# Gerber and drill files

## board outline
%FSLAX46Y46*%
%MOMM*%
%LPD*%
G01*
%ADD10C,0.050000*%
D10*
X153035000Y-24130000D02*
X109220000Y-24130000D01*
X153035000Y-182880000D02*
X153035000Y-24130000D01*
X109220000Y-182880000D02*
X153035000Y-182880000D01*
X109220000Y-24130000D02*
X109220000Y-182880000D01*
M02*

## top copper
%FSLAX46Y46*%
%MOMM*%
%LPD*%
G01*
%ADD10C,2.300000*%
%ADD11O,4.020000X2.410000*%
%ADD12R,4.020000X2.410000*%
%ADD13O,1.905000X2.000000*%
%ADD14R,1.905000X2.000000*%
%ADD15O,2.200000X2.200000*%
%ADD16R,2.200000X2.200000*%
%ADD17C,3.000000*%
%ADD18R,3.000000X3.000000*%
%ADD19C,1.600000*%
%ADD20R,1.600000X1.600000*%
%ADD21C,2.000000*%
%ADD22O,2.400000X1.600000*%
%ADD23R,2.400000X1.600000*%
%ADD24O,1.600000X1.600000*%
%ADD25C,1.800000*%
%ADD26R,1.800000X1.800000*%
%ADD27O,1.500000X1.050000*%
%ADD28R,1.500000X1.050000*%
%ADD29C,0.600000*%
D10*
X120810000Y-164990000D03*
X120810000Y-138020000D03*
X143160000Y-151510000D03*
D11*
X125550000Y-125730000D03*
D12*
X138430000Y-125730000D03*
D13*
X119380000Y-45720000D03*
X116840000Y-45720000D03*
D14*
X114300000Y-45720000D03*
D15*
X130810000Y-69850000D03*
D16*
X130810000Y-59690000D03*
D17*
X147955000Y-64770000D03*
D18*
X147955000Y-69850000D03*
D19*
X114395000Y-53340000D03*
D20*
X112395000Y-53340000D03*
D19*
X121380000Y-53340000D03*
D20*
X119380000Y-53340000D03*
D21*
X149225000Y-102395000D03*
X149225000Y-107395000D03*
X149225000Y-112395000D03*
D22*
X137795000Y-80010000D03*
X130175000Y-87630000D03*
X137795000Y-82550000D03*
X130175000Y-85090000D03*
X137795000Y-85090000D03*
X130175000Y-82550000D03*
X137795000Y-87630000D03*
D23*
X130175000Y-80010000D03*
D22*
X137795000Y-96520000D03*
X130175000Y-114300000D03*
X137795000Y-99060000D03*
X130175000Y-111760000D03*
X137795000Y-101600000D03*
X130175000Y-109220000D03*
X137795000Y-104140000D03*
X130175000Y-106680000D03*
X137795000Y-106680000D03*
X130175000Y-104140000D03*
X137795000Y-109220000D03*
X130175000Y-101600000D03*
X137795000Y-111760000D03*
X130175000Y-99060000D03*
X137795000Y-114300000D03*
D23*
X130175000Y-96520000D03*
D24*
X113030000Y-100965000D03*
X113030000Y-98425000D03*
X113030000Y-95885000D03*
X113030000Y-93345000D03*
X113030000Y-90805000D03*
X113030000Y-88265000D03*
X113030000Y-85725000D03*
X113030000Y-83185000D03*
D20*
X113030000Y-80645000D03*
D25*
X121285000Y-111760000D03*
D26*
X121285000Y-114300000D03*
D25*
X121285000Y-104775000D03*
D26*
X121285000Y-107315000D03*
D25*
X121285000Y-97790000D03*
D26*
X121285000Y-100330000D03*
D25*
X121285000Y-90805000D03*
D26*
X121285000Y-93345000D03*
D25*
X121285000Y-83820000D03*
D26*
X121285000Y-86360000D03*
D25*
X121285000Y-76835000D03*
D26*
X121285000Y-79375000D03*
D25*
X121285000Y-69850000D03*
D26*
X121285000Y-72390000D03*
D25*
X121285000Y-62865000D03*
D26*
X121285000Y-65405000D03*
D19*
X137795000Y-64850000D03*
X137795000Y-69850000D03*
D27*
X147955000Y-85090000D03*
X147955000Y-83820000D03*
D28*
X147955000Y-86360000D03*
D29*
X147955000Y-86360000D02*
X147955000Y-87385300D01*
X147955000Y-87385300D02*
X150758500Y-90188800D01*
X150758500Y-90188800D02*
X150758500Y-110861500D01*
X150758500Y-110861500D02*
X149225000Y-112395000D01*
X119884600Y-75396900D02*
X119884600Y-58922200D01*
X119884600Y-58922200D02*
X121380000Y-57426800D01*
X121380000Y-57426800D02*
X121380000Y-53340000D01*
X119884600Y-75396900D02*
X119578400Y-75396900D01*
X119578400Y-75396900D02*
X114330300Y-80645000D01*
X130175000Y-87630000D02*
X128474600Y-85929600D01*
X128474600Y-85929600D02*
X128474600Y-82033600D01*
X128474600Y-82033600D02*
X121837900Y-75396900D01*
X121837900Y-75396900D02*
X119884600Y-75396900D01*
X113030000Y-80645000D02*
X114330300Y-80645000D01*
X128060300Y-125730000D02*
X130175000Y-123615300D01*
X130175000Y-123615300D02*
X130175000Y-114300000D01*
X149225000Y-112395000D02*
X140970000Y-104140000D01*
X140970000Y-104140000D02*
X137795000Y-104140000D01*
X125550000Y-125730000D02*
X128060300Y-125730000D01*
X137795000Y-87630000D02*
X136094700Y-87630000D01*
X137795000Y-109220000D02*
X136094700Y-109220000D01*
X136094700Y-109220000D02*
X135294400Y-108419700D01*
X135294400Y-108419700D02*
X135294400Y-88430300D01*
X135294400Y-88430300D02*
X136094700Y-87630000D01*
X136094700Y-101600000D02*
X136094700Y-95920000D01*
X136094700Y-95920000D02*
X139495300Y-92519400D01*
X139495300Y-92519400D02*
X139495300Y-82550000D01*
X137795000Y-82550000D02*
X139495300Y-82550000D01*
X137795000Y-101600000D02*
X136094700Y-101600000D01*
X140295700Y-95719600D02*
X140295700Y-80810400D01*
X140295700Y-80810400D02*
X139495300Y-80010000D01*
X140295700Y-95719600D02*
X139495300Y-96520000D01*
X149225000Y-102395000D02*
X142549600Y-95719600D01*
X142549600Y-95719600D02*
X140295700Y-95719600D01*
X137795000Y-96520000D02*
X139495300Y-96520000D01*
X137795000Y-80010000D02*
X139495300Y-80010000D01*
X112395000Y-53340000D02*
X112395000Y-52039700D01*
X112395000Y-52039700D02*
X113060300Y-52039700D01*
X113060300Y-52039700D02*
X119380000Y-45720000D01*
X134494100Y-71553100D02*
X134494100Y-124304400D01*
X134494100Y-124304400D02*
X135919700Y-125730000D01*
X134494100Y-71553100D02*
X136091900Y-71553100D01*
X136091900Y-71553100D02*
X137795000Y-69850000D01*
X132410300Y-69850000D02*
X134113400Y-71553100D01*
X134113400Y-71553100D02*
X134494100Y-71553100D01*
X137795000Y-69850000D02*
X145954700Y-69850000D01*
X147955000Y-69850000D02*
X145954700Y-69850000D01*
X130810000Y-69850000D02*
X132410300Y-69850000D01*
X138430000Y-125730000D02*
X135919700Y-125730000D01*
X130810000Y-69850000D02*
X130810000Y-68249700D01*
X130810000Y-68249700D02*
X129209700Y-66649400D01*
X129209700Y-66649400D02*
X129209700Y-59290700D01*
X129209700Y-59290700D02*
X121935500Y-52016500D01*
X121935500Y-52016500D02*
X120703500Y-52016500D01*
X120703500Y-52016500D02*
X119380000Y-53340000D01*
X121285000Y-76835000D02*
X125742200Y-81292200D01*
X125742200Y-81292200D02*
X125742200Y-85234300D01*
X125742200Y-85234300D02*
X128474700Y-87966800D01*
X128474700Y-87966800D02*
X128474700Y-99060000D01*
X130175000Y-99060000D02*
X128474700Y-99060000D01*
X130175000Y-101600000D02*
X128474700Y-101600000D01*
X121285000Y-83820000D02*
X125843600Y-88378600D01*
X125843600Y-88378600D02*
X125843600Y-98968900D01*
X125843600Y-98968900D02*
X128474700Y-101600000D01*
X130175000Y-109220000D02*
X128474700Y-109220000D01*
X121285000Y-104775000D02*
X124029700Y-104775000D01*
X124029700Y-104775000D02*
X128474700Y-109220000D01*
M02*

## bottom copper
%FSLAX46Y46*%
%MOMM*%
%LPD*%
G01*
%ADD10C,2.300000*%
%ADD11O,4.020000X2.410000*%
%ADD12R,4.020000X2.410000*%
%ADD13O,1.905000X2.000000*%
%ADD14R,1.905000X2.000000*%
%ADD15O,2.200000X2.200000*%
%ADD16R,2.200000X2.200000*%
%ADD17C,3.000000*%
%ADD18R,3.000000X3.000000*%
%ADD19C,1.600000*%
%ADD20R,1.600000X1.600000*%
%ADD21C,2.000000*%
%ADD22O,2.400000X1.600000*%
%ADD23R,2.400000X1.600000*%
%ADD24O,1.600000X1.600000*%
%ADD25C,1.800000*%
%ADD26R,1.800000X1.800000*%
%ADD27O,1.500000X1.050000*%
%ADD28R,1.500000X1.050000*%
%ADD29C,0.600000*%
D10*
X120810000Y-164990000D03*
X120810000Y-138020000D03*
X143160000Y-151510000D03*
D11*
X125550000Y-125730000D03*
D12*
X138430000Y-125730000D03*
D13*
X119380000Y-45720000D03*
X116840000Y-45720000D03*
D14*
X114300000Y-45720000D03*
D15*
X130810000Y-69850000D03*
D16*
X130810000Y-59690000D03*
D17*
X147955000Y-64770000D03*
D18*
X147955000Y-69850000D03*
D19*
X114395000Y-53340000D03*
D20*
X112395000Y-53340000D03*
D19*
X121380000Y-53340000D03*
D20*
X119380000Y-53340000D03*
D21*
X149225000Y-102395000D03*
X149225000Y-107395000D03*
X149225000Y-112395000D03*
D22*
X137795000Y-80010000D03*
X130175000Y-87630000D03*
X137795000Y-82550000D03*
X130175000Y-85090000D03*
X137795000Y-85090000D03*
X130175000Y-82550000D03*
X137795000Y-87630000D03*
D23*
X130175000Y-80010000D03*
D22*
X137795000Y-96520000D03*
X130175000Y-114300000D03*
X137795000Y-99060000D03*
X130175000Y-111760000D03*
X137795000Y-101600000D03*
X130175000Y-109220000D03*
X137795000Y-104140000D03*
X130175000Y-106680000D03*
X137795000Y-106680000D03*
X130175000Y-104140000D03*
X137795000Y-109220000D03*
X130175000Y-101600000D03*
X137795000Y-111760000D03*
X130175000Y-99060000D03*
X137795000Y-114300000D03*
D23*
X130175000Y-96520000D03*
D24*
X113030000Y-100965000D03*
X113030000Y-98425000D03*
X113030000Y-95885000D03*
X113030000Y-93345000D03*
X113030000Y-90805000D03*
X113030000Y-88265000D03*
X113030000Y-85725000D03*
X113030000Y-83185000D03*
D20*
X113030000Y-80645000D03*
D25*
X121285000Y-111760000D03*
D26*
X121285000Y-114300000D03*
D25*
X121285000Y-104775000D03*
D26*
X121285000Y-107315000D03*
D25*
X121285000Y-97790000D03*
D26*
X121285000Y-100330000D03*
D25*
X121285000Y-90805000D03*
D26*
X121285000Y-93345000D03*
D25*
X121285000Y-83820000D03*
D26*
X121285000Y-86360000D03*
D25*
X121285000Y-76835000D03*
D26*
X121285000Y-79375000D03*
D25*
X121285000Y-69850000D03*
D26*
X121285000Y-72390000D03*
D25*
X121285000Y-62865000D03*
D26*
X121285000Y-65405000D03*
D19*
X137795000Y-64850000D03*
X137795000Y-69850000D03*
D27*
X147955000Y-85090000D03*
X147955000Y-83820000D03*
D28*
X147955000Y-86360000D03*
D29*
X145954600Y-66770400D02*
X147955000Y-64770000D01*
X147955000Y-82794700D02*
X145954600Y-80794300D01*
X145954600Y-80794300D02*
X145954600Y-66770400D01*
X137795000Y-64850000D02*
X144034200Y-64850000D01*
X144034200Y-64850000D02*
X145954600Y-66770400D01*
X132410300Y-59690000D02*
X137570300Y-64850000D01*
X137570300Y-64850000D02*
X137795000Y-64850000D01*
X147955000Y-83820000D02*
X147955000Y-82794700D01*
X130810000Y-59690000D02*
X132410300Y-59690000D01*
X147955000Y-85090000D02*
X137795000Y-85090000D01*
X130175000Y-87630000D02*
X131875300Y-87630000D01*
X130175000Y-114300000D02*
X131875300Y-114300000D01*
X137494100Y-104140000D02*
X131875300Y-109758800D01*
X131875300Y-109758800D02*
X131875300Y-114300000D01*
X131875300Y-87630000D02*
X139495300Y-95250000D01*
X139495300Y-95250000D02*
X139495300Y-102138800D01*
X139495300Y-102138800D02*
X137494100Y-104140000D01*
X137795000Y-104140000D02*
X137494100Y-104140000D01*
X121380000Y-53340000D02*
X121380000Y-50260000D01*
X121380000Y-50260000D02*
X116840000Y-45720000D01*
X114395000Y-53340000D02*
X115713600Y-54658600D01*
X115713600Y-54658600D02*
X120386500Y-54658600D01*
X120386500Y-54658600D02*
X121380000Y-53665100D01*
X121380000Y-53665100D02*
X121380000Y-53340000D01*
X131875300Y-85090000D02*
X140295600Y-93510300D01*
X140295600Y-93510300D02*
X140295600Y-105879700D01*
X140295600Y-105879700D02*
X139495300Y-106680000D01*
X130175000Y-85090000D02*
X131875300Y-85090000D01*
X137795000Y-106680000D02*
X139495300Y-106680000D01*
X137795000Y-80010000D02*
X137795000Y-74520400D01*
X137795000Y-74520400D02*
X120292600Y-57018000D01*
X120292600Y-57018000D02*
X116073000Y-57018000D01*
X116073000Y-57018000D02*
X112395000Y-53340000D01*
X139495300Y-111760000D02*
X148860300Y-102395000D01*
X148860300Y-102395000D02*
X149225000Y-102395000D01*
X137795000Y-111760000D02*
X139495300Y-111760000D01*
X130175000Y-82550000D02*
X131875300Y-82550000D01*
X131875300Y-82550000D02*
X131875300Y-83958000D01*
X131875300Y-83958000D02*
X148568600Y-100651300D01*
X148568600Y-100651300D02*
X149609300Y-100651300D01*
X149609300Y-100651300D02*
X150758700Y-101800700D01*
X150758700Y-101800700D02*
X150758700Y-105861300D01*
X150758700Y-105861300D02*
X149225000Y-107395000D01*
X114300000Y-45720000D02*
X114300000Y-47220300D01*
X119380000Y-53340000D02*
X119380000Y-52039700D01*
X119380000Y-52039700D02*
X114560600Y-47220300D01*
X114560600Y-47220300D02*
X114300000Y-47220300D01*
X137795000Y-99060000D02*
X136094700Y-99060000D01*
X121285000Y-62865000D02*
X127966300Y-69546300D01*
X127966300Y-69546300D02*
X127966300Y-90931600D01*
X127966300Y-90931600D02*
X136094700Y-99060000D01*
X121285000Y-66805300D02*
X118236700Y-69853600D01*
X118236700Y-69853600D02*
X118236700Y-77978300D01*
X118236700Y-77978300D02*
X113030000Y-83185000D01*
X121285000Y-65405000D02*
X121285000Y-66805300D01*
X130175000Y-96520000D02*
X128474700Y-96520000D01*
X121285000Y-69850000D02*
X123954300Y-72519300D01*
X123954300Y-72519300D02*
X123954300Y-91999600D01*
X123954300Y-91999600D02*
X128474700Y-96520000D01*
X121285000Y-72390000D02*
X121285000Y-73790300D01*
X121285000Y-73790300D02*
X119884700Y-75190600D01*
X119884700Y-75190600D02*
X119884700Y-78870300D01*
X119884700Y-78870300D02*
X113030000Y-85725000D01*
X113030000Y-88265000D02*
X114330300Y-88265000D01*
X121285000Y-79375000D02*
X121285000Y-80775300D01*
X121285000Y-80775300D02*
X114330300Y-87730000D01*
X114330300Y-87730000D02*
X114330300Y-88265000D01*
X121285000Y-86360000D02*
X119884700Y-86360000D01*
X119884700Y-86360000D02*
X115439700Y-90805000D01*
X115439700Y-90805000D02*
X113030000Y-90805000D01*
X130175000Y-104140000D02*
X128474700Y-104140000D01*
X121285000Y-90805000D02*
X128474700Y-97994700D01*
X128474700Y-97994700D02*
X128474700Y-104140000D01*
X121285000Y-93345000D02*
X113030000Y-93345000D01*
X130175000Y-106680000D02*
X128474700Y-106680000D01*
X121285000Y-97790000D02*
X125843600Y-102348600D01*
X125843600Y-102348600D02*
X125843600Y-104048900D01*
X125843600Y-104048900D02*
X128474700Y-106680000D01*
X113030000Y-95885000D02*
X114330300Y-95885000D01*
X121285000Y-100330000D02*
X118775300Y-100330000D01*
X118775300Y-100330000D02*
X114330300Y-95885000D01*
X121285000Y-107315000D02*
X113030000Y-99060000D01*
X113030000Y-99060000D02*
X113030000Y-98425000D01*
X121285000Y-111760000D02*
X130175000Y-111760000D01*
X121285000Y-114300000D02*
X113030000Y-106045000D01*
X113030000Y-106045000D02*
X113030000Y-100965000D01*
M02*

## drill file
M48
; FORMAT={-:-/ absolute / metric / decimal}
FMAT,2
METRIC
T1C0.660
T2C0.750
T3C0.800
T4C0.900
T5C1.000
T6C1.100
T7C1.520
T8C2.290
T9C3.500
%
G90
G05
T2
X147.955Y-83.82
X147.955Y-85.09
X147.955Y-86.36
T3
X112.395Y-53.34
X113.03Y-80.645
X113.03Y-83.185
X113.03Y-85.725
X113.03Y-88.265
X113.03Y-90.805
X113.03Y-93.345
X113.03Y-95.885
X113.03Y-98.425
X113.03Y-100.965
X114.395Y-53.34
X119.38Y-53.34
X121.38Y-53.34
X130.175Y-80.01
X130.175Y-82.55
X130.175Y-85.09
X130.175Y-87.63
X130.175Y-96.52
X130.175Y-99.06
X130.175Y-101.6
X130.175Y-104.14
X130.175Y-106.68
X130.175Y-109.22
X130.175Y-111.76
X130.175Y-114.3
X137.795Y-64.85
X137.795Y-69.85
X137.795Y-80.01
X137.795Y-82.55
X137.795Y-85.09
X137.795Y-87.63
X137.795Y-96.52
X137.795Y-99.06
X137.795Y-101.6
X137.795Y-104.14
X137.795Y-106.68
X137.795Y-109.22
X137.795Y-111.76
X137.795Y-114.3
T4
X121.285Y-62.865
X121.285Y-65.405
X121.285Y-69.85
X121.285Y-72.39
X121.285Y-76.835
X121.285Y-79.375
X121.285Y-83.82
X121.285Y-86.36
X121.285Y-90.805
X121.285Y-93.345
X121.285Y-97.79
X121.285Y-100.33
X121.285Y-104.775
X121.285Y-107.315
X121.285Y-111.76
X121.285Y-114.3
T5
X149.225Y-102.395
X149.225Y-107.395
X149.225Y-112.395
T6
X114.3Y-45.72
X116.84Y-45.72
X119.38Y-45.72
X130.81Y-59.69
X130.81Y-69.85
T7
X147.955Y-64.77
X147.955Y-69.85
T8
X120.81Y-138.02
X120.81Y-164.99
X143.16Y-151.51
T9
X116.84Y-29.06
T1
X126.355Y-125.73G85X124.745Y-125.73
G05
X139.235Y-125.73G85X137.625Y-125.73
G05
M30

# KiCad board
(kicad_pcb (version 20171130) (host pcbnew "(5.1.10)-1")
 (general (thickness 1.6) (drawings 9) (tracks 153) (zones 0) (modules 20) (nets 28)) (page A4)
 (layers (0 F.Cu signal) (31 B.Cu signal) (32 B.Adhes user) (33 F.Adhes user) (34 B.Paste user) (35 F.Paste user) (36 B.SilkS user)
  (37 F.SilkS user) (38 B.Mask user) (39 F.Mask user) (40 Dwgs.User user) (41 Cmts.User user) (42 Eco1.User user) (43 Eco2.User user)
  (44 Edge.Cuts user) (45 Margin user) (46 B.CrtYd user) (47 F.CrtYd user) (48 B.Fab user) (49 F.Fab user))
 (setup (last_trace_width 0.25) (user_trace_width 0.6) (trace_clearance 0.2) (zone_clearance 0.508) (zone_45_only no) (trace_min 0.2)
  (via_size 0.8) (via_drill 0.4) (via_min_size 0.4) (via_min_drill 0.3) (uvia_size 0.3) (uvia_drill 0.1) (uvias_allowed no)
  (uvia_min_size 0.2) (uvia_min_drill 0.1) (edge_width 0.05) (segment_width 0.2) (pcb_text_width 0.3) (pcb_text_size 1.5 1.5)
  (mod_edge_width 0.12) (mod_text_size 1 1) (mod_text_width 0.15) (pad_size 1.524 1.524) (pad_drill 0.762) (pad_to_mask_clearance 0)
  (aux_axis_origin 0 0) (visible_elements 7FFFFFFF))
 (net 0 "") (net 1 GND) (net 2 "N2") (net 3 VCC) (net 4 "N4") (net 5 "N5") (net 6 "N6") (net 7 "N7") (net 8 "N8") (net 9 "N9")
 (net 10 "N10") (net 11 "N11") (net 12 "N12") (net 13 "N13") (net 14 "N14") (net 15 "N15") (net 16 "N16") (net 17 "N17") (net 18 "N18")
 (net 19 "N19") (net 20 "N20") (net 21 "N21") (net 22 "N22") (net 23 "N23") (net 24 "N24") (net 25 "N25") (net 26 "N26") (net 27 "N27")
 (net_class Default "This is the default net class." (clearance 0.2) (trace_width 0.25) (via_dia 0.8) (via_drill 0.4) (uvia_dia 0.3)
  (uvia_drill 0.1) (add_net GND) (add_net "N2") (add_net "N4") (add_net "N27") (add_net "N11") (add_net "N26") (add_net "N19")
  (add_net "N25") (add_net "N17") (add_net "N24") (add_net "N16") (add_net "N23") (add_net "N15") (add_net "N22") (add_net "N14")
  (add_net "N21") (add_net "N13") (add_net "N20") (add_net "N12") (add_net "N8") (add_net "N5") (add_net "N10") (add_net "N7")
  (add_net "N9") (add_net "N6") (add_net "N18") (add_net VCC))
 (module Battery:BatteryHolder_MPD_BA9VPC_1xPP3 (layer F.Cu) (at 138.43 125.73 270)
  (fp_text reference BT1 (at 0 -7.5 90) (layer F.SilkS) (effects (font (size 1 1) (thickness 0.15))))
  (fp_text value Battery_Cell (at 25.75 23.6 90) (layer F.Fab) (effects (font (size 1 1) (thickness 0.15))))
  (pad "" np_thru_hole circle (at 39.26 17.62 270) (size 2.3 2.3) (drill 2.29) (layers *.Cu *.Mask))
  (pad "" np_thru_hole circle (at 12.29 17.62 270) (size 2.3 2.3) (drill 2.29) (layers *.Cu *.Mask))
  (pad "" np_thru_hole circle (at 25.78 -4.73 270) (size 2.3 2.3) (drill 2.29) (layers *.Cu *.Mask))
  (pad 2 thru_hole oval (at 0 12.88 270) (size 2.41 4.02) (drill oval 0.66 2.27) (layers *.Cu *.Mask) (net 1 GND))
  (pad 1 thru_hole rect (at 0 0 270) (size 2.41 4.02) (drill oval 0.66 2.27) (layers *.Cu *.Mask) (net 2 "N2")))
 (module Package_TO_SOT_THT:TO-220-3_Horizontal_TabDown (layer F.Cu) (at 114.3 45.72)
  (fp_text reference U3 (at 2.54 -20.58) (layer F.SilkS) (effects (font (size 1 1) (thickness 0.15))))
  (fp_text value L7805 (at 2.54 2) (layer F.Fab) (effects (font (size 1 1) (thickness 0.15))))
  (pad 3 thru_hole oval (at 5.08 0) (size 1.905 2) (drill 1.1) (layers *.Cu *.Mask) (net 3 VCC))
  (pad 2 thru_hole oval (at 2.54 0) (size 1.905 2) (drill 1.1) (layers *.Cu *.Mask) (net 1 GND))
  (pad 1 thru_hole rect (at 0 0) (size 1.905 2) (drill 1.1) (layers *.Cu *.Mask) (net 2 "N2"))
  (pad "" np_thru_hole oval (at 2.54 -16.66) (size 3.5 3.5) (drill 3.5) (layers *.Cu *.Mask)))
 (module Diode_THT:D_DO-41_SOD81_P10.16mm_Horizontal (layer F.Cu) (at 130.81 59.69 270)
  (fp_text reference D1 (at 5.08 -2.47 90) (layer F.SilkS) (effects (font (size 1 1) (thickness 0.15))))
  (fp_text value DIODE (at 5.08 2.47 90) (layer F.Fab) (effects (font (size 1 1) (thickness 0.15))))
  (pad 2 thru_hole oval (at 10.16 0 270) (size 2.2 2.2) (drill 1.1) (layers *.Cu *.Mask) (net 2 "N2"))
  (pad 1 thru_hole rect (at 0 0 270) (size 2.2 2.2) (drill 1.1) (layers *.Cu *.Mask) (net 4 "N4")))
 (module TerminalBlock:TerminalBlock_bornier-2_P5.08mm (layer F.Cu) (at 147.955 69.85 90)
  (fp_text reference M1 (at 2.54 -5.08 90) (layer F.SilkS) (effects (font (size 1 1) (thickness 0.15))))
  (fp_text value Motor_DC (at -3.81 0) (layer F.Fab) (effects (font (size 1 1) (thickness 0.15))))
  (pad 2 thru_hole circle (at 5.08 0 90) (size 3 3) (drill 1.52) (layers *.Cu *.Mask) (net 4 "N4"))
  (pad 1 thru_hole rect (at 0 0 90) (size 3 3) (drill 1.52) (layers *.Cu *.Mask) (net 2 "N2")))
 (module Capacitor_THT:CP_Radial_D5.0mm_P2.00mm (layer F.Cu) (at 112.395 53.34)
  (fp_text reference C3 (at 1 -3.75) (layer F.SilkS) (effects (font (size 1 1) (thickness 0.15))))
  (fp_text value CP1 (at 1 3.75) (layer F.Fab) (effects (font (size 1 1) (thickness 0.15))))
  (pad 2 thru_hole circle (at 2 0) (size 1.6 1.6) (drill 0.8) (layers *.Cu *.Mask) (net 1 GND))
  (pad 1 thru_hole rect (at 0 0) (size 1.6 1.6) (drill 0.8) (layers *.Cu *.Mask) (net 3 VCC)))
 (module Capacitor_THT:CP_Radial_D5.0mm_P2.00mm (layer F.Cu) (at 119.38 53.34)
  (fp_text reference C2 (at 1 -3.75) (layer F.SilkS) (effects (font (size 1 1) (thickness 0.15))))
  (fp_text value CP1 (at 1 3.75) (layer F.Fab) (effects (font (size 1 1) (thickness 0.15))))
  (pad 2 thru_hole circle (at 2 0) (size 1.6 1.6) (drill 0.8) (layers *.Cu *.Mask) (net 1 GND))
  (pad 1 thru_hole rect (at 0 0) (size 1.6 1.6) (drill 0.8) (layers *.Cu *.Mask) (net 2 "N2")))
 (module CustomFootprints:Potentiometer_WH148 (layer F.Cu) (at 140.335 107.395 90)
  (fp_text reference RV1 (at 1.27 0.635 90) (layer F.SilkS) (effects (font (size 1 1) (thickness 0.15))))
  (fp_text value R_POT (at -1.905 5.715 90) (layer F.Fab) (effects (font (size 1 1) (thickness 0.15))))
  (pad 3 thru_hole circle (at 5 8.89 90) (size 2 2) (drill 1) (layers *.Cu *.Mask) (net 3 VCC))
  (pad 2 thru_hole circle (at 0 8.89 90) (size 2 2) (drill 1) (layers *.Cu *.Mask) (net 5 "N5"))
  (pad 1 thru_hole circle (at -5 8.89 90) (size 2 2) (drill 1) (layers *.Cu *.Mask) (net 1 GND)))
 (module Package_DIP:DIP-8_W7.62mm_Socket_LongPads (layer F.Cu) (at 130.175 80.01)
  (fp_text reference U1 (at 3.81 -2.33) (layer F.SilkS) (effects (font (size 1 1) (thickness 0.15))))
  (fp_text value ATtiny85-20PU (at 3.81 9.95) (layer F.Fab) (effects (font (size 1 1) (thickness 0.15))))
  (pad 8 thru_hole oval (at 7.62 0) (size 2.4 1.6) (drill 0.8) (layers *.Cu *.Mask) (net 3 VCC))
  (pad 4 thru_hole oval (at 0 7.62) (size 2.4 1.6) (drill 0.8) (layers *.Cu *.Mask) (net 1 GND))
  (pad 7 thru_hole oval (at 7.62 2.54) (size 2.4 1.6) (drill 0.8) (layers *.Cu *.Mask) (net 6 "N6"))
  (pad 3 thru_hole oval (at 0 5.08) (size 2.4 1.6) (drill 0.8) (layers *.Cu *.Mask) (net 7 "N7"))
  (pad 6 thru_hole oval (at 7.62 5.08) (size 2.4 1.6) (drill 0.8) (layers *.Cu *.Mask) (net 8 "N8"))
  (pad 2 thru_hole oval (at 0 2.54) (size 2.4 1.6) (drill 0.8) (layers *.Cu *.Mask) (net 5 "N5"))
  (pad 5 thru_hole oval (at 7.62 7.62) (size 2.4 1.6) (drill 0.8) (layers *.Cu *.Mask) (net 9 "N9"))
  (pad 1 thru_hole rect (at 0 0) (size 2.4 1.6) (drill 0.8) (layers *.Cu *.Mask) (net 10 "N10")))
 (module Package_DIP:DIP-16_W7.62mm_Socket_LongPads (layer F.Cu) (at 130.175 96.52)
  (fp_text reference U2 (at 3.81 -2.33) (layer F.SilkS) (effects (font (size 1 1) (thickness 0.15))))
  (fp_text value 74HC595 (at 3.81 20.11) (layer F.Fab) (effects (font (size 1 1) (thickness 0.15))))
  (pad 16 thru_hole oval (at 7.62 0) (size 2.4 1.6) (drill 0.8) (layers *.Cu *.Mask) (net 3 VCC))
  (pad 8 thru_hole oval (at 0 17.78) (size 2.4 1.6) (drill 0.8) (layers *.Cu *.Mask) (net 1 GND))
  (pad 15 thru_hole oval (at 7.62 2.54) (size 2.4 1.6) (drill 0.8) (layers *.Cu *.Mask) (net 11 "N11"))
  (pad 7 thru_hole oval (at 0 15.24) (size 2.4 1.6) (drill 0.8) (layers *.Cu *.Mask) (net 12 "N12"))
  (pad 14 thru_hole oval (at 7.62 5.08) (size 2.4 1.6) (drill 0.8) (layers *.Cu *.Mask) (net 6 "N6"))
  (pad 6 thru_hole oval (at 0 12.7) (size 2.4 1.6) (drill 0.8) (layers *.Cu *.Mask) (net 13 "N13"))
  (pad 13 thru_hole oval (at 7.62 7.62) (size 2.4 1.6) (drill 0.8) (layers *.Cu *.Mask) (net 1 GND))
  (pad 5 thru_hole oval (at 0 10.16) (size 2.4 1.6) (drill 0.8) (layers *.Cu *.Mask) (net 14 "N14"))
  (pad 12 thru_hole oval (at 7.62 10.16) (size 2.4 1.6) (drill 0.8) (layers *.Cu *.Mask) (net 7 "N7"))
  (pad 4 thru_hole oval (at 0 7.62) (size 2.4 1.6) (drill 0.8) (layers *.Cu *.Mask) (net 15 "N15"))
  (pad 11 thru_hole oval (at 7.62 12.7) (size 2.4 1.6) (drill 0.8) (layers *.Cu *.Mask) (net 9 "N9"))
  (pad 3 thru_hole oval (at 0 5.08) (size 2.4 1.6) (drill 0.8) (layers *.Cu *.Mask) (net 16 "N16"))
  (pad 10 thru_hole oval (at 7.62 15.24) (size 2.4 1.6) (drill 0.8) (layers *.Cu *.Mask) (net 3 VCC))
  (pad 2 thru_hole oval (at 0 2.54) (size 2.4 1.6) (drill 0.8) (layers *.Cu *.Mask) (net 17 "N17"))
  (pad 9 thru_hole oval (at 7.62 17.78) (size 2.4 1.6) (drill 0.8) (layers *.Cu *.Mask) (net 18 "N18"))
  (pad 1 thru_hole rect (at 0 0) (size 2.4 1.6) (drill 0.8) (layers *.Cu *.Mask) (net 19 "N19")))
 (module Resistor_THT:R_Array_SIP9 (layer F.Cu) (at 113.03 80.645 270)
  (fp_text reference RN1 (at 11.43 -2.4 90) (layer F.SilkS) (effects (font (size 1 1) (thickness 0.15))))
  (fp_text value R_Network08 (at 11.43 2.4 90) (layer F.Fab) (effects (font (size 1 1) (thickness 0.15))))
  (pad 9 thru_hole oval (at 20.32 0 270) (size 1.6 1.6) (drill 0.8) (layers *.Cu *.Mask) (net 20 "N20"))
  (pad 8 thru_hole oval (at 17.78 0 270) (size 1.6 1.6) (drill 0.8) (layers *.Cu *.Mask) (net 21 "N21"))
  (pad 7 thru_hole oval (at 15.24 0 270) (size 1.6 1.6) (drill 0.8) (layers *.Cu *.Mask) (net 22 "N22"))
  (pad 6 thru_hole oval (at 12.7 0 270) (size 1.6 1.6) (drill 0.8) (layers *.Cu *.Mask) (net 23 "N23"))
  (pad 5 thru_hole oval (at 10.16 0 270) (size 1.6 1.6) (drill 0.8) (layers *.Cu *.Mask) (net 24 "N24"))
  (pad 4 thru_hole oval (at 7.62 0 270) (size 1.6 1.6) (drill 0.8) (layers *.Cu *.Mask) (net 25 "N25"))
  (pad 3 thru_hole oval (at 5.08 0 270) (size 1.6 1.6) (drill 0.8) (layers *.Cu *.Mask) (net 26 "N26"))
  (pad 2 thru_hole oval (at 2.54 0 270) (size 1.6 1.6) (drill 0.8) (layers *.Cu *.Mask) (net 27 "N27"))
  (pad 1 thru_hole rect (at 0 0 270) (size 1.6 1.6) (drill 0.8) (layers *.Cu *.Mask) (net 1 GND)))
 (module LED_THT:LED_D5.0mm (layer F.Cu) (at 121.285 114.3 90)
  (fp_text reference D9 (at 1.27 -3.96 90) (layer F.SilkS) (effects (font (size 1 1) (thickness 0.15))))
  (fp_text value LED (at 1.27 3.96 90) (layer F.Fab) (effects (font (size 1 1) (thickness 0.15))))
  (pad 2 thru_hole circle (at 2.54 0 90) (size 1.8 1.8) (drill 0.9) (layers *.Cu *.Mask) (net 12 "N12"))
  (pad 1 thru_hole rect (at 0 0 90) (size 1.8 1.8) (drill 0.9) (layers *.Cu *.Mask) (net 20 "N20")))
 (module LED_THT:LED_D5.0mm (layer F.Cu) (at 121.285 107.315 90)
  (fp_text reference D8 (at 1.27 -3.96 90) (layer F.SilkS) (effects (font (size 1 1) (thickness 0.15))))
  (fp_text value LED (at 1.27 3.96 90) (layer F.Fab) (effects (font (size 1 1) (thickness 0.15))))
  (pad 2 thru_hole circle (at 2.54 0 90) (size 1.8 1.8) (drill 0.9) (layers *.Cu *.Mask) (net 13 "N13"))
  (pad 1 thru_hole rect (at 0 0 90) (size 1.8 1.8) (drill 0.9) (layers *.Cu *.Mask) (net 21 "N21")))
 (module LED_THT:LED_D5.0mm (layer F.Cu) (at 121.285 100.33 90)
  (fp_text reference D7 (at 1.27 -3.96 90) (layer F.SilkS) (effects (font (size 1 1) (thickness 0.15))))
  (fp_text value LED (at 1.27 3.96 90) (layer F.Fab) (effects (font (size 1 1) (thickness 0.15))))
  (pad 2 thru_hole circle (at 2.54 0 90) (size 1.8 1.8) (drill 0.9) (layers *.Cu *.Mask) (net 14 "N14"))
  (pad 1 thru_hole rect (at 0 0 90) (size 1.8 1.8) (drill 0.9) (layers *.Cu *.Mask) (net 22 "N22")))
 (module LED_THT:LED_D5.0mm (layer F.Cu) (at 121.285 93.345 90)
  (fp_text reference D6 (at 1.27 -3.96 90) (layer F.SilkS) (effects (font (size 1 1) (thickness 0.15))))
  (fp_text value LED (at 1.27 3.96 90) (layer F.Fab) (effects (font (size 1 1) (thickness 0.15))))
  (pad 2 thru_hole circle (at 2.54 0 90) (size 1.8 1.8) (drill 0.9) (layers *.Cu *.Mask) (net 15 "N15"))
  (pad 1 thru_hole rect (at 0 0 90) (size 1.8 1.8) (drill 0.9) (layers *.Cu *.Mask) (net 23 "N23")))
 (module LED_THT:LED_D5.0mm (layer F.Cu) (at 121.285 86.36 90)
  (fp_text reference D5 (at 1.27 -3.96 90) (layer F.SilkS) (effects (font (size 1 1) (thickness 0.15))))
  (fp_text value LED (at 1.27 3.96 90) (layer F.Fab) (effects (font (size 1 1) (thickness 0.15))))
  (pad 2 thru_hole circle (at 2.54 0 90) (size 1.8 1.8) (drill 0.9) (layers *.Cu *.Mask) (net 16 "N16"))
  (pad 1 thru_hole rect (at 0 0 90) (size 1.8 1.8) (drill 0.9) (layers *.Cu *.Mask) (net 24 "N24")))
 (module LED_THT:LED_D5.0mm (layer F.Cu) (at 121.285 79.375 90)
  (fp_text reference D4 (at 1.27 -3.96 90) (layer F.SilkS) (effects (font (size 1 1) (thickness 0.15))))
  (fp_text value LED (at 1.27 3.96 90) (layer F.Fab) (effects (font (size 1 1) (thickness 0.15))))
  (pad 2 thru_hole circle (at 2.54 0 90) (size 1.8 1.8) (drill 0.9) (layers *.Cu *.Mask) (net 17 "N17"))
  (pad 1 thru_hole rect (at 0 0 90) (size 1.8 1.8) (drill 0.9) (layers *.Cu *.Mask) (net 25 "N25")))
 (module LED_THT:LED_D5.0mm (layer F.Cu) (at 121.285 72.39 90)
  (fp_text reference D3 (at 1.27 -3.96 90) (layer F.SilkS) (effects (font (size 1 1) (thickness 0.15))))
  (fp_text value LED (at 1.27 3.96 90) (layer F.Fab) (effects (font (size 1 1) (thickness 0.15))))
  (pad 2 thru_hole circle (at 2.54 0 90) (size 1.8 1.8) (drill 0.9) (layers *.Cu *.Mask) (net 19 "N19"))
  (pad 1 thru_hole rect (at 0 0 90) (size 1.8 1.8) (drill 0.9) (layers *.Cu *.Mask) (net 26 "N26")))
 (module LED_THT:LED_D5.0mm (layer F.Cu) (at 121.285 65.405 90)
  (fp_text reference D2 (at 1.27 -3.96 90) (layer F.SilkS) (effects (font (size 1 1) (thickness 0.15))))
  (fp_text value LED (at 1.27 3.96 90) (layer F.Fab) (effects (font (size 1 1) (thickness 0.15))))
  (pad 2 thru_hole circle (at 2.54 0 90) (size 1.8 1.8) (drill 0.9) (layers *.Cu *.Mask) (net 11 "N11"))
  (pad 1 thru_hole rect (at 0 0 90) (size 1.8 1.8) (drill 0.9) (layers *.Cu *.Mask) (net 27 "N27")))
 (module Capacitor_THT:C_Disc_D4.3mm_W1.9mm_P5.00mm (layer F.Cu) (at 137.795 69.85 90)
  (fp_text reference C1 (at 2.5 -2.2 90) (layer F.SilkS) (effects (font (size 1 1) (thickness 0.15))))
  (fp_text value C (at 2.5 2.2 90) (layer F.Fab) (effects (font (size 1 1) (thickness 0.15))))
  (pad 2 thru_hole circle (at 5 0 90) (size 1.6 1.6) (drill 0.8) (layers *.Cu *.Mask) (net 4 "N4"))
  (pad 1 thru_hole circle (at 0 0 90) (size 1.6 1.6) (drill 0.8) (layers *.Cu *.Mask) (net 2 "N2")))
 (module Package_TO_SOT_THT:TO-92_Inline (layer F.Cu) (at 147.955 86.36 90)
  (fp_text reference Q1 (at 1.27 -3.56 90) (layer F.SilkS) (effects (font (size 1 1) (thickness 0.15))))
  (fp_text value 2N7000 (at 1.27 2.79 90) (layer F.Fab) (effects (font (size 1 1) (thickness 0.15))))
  (pad 2 thru_hole oval (at 1.27 0 90) (size 1.05 1.5) (drill 0.75) (layers *.Cu *.Mask) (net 8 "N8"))
  (pad 3 thru_hole oval (at 2.54 0 90) (size 1.05 1.5) (drill 0.75) (layers *.Cu *.Mask) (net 4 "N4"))
  (pad 1 thru_hole rect (at 0 0 90) (size 1.05 1.5) (drill 0.75) (layers *.Cu *.Mask) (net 1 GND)))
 (gr_line (start 153.035 24.13) (end 109.22 24.13) (layer Edge.Cuts) (width 0.05))
 (gr_line (start 153.035 182.88) (end 153.035 24.13) (layer Edge.Cuts) (width 0.05))
 (gr_line (start 109.22 182.88) (end 153.035 182.88) (layer Edge.Cuts) (width 0.05))
 (gr_line (start 109.22 24.13) (end 109.22 182.88) (layer Edge.Cuts) (width 0.05))
 (segment (start 145.9546 66.7704) (end 147.955 64.77) (width 0.6) (layer B.Cu) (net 4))
 (segment (start 147.955 82.7947) (end 145.9546 80.7943) (width 0.6) (layer B.Cu) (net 4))
 (segment (start 145.9546 80.7943) (end 145.9546 66.7704) (width 0.6) (layer B.Cu) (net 4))
 (segment (start 137.795 64.85) (end 144.0342 64.85) (width 0.6) (layer B.Cu) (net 4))
 (segment (start 144.0342 64.85) (end 145.9546 66.7704) (width 0.6) (layer B.Cu) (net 4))
 (segment (start 132.4103 59.69) (end 137.5703 64.85) (width 0.6) (layer B.Cu) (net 4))
 (segment (start 137.5703 64.85) (end 137.795 64.85) (width 0.6) (layer B.Cu) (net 4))
 (segment (start 147.955 83.82) (end 147.955 82.7947) (width 0.6) (layer B.Cu) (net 4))
 (segment (start 130.81 59.69) (end 132.4103 59.69) (width 0.6) (layer B.Cu) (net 4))
 (segment (start 147.955 85.09) (end 137.795 85.09) (width 0.6) (layer B.Cu) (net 8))
 (segment (start 147.955 86.36) (end 147.955 87.3853) (width 0.6) (layer F.Cu) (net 1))
 (segment (start 147.955 87.3853) (end 150.7585 90.1888) (width 0.6) (layer F.Cu) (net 1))
 (segment (start 150.7585 90.1888) (end 150.7585 110.8615) (width 0.6) (layer F.Cu) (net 1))
 (segment (start 150.7585 110.8615) (end 149.225 112.395) (width 0.6) (layer F.Cu) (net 1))
 (segment (start 119.8846 75.3969) (end 119.8846 58.9222) (width 0.6) (layer F.Cu) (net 1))
 (segment (start 119.8846 58.9222) (end 121.38 57.4268) (width 0.6) (layer F.Cu) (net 1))
 (segment (start 121.38 57.4268) (end 121.38 53.34) (width 0.6) (layer F.Cu) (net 1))
 (segment (start 119.8846 75.3969) (end 119.5784 75.3969) (width 0.6) (layer F.Cu) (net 1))
 (segment (start 119.5784 75.3969) (end 114.3303 80.645) (width 0.6) (layer F.Cu) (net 1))
 (segment (start 130.175 87.63) (end 128.4746 85.9296) (width 0.6) (layer F.Cu) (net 1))
 (segment (start 128.4746 85.9296) (end 128.4746 82.0336) (width 0.6) (layer F.Cu) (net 1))
 (segment (start 128.4746 82.0336) (end 121.8379 75.3969) (width 0.6) (layer F.Cu) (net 1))
 (segment (start 121.8379 75.3969) (end 119.8846 75.3969) (width 0.6) (layer F.Cu) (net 1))
 (segment (start 113.03 80.645) (end 114.3303 80.645) (width 0.6) (layer F.Cu) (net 1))
 (segment (start 130.175 87.63) (end 131.8753 87.63) (width 0.6) (layer B.Cu) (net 1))
 (segment (start 130.175 114.3) (end 131.8753 114.3) (width 0.6) (layer B.Cu) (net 1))
 (segment (start 137.4941 104.14) (end 131.8753 109.7588) (width 0.6) (layer B.Cu) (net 1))
 (segment (start 131.8753 109.7588) (end 131.8753 114.3) (width 0.6) (layer B.Cu) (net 1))
 (segment (start 131.8753 87.63) (end 139.4953 95.25) (width 0.6) (layer B.Cu) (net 1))
 (segment (start 139.4953 95.25) (end 139.4953 102.1388) (width 0.6) (layer B.Cu) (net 1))
 (segment (start 139.4953 102.1388) (end 137.4941 104.14) (width 0.6) (layer B.Cu) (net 1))
 (segment (start 137.795 104.14) (end 137.4941 104.14) (width 0.6) (layer B.Cu) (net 1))
 (segment (start 128.0603 125.73) (end 130.175 123.6153) (width 0.6) (layer F.Cu) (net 1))
 (segment (start 130.175 123.6153) (end 130.175 114.3) (width 0.6) (layer F.Cu) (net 1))
 (segment (start 149.225 112.395) (end 140.97 104.14) (width 0.6) (layer F.Cu) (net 1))
 (segment (start 140.97 104.14) (end 137.795 104.14) (width 0.6) (layer F.Cu) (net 1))
 (segment (start 125.55 125.73) (end 128.0603 125.73) (width 0.6) (layer F.Cu) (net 1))
 (segment (start 121.38 53.34) (end 121.38 50.26) (width 0.6) (layer B.Cu) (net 1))
 (segment (start 121.38 50.26) (end 116.84 45.72) (width 0.6) (layer B.Cu) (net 1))
 (segment (start 114.395 53.34) (end 115.7136 54.6586) (width 0.6) (layer B.Cu) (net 1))
 (segment (start 115.7136 54.6586) (end 120.3865 54.6586) (width 0.6) (layer B.Cu) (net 1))
 (segment (start 120.3865 54.6586) (end 121.38 53.6651) (width 0.6) (layer B.Cu) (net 1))
 (segment (start 121.38 53.6651) (end 121.38 53.34) (width 0.6) (layer B.Cu) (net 1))
 (segment (start 137.795 87.63) (end 136.0947 87.63) (width 0.6) (layer F.Cu) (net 9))
 (segment (start 137.795 109.22) (end 136.0947 109.22) (width 0.6) (layer F.Cu) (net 9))
 (segment (start 136.0947 109.22) (end 135.2944 108.4197) (width 0.6) (layer F.Cu) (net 9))
 (segment (start 135.2944 108.4197) (end 135.2944 88.4303) (width 0.6) (layer F.Cu) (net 9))
 (segment (start 135.2944 88.4303) (end 136.0947 87.63) (width 0.6) (layer F.Cu) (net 9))
 (segment (start 131.8753 85.09) (end 140.2956 93.5103) (width 0.6) (layer B.Cu) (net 7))
 (segment (start 140.2956 93.5103) (end 140.2956 105.8797) (width 0.6) (layer B.Cu) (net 7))
 (segment (start 140.2956 105.8797) (end 139.4953 106.68) (width 0.6) (layer B.Cu) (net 7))
 (segment (start 130.175 85.09) (end 131.8753 85.09) (width 0.6) (layer B.Cu) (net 7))
 (segment (start 137.795 106.68) (end 139.4953 106.68) (width 0.6) (layer B.Cu) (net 7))
 (segment (start 136.0947 101.6) (end 136.0947 95.92) (width 0.6) (layer F.Cu) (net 6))
 (segment (start 136.0947 95.92) (end 139.4953 92.5194) (width 0.6) (layer F.Cu) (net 6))
 (segment (start 139.4953 92.5194) (end 139.4953 82.55) (width 0.6) (layer F.Cu) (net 6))
 (segment (start 137.795 82.55) (end 139.4953 82.55) (width 0.6) (layer F.Cu) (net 6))
 (segment (start 137.795 101.6) (end 136.0947 101.6) (width 0.6) (layer F.Cu) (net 6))
 (segment (start 140.2957 95.7196) (end 140.2957 80.8104) (width 0.6) (layer F.Cu) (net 3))
 (segment (start 140.2957 80.8104) (end 139.4953 80.01) (width 0.6) (layer F.Cu) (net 3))
 (segment (start 137.795 80.01) (end 137.795 74.5204) (width 0.6) (layer B.Cu) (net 3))
 (segment (start 137.795 74.5204) (end 120.2926 57.018) (width 0.6) (layer B.Cu) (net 3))
 (segment (start 120.2926 57.018) (end 116.073 57.018) (width 0.6) (layer B.Cu) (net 3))
 (segment (start 116.073 57.018) (end 112.395 53.34) (width 0.6) (layer B.Cu) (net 3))
 (segment (start 140.2957 95.7196) (end 139.4953 96.52) (width 0.6) (layer F.Cu) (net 3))
 (segment (start 149.225 102.395) (end 142.5496 95.7196) (width 0.6) (layer F.Cu) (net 3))
 (segment (start 142.5496 95.7196) (end 140.2957 95.7196) (width 0.6) (layer F.Cu) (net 3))
 (segment (start 137.795 96.52) (end 139.4953 96.52) (width 0.6) (layer F.Cu) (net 3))
 (segment (start 139.4953 111.76) (end 148.8603 102.395) (width 0.6) (layer B.Cu) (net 3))
 (segment (start 148.8603 102.395) (end 149.225 102.395) (width 0.6) (layer B.Cu) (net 3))
 (segment (start 137.795 80.01) (end 139.4953 80.01) (width 0.6) (layer F.Cu) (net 3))
 (segment (start 112.395 53.34) (end 112.395 52.0397) (width 0.6) (layer F.Cu) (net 3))
 (segment (start 112.395 52.0397) (end 113.0603 52.0397) (width 0.6) (layer F.Cu) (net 3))
 (segment (start 113.0603 52.0397) (end 119.38 45.72) (width 0.6) (layer F.Cu) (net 3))
 (segment (start 137.795 111.76) (end 139.4953 111.76) (width 0.6) (layer B.Cu) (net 3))
 (segment (start 130.175 82.55) (end 131.8753 82.55) (width 0.6) (layer B.Cu) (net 5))
 (segment (start 131.8753 82.55) (end 131.8753 83.958) (width 0.6) (layer B.Cu) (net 5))
 (segment (start 131.8753 83.958) (end 148.5686 100.6513) (width 0.6) (layer B.Cu) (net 5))
 (segment (start 148.5686 100.6513) (end 149.6093 100.6513) (width 0.6) (layer B.Cu) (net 5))
 (segment (start 149.6093 100.6513) (end 150.7587 101.8007) (width 0.6) (layer B.Cu) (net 5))
 (segment (start 150.7587 101.8007) (end 150.7587 105.8613) (width 0.6) (layer B.Cu) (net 5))
 (segment (start 150.7587 105.8613) (end 149.225 107.395) (width 0.6) (layer B.Cu) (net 5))
 (segment (start 134.4941 71.5531) (end 134.4941 124.3044) (width 0.6) (layer F.Cu) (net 2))
 (segment (start 134.4941 124.3044) (end 135.9197 125.73) (width 0.6) (layer F.Cu) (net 2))
 (segment (start 134.4941 71.5531) (end 136.0919 71.5531) (width 0.6) (layer F.Cu) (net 2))
 (segment (start 136.0919 71.5531) (end 137.795 69.85) (width 0.6) (layer F.Cu) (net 2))
 (segment (start 132.4103 69.85) (end 134.1134 71.5531) (width 0.6) (layer F.Cu) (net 2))
 (segment (start 134.1134 71.5531) (end 134.4941 71.5531) (width 0.6) (layer F.Cu) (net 2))
 (segment (start 137.795 69.85) (end 145.9547 69.85) (width 0.6) (layer F.Cu) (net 2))
 (segment (start 147.955 69.85) (end 145.9547 69.85) (width 0.6) (layer F.Cu) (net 2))
 (segment (start 130.81 69.85) (end 132.4103 69.85) (width 0.6) (layer F.Cu) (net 2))
 (segment (start 138.43 125.73) (end 135.9197 125.73) (width 0.6) (layer F.Cu) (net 2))
 (segment (start 130.81 69.85) (end 130.81 68.2497) (width 0.6) (layer F.Cu) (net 2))
 (segment (start 130.81 68.2497) (end 129.2097 66.6494) (width 0.6) (layer F.Cu) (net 2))
 (segment (start 129.2097 66.6494) (end 129.2097 59.2907) (width 0.6) (layer F.Cu) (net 2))
 (segment (start 129.2097 59.2907) (end 121.9355 52.0165) (width 0.6) (layer F.Cu) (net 2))
 (segment (start 121.9355 52.0165) (end 120.7035 52.0165) (width 0.6) (layer F.Cu) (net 2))
 (segment (start 120.7035 52.0165) (end 119.38 53.34) (width 0.6) (layer F.Cu) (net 2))
 (segment (start 114.3 45.72) (end 114.3 47.2203) (width 0.6) (layer B.Cu) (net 2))
 (segment (start 119.38 53.34) (end 119.38 52.0397) (width 0.6) (layer B.Cu) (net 2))
 (segment (start 119.38 52.0397) (end 114.5606 47.2203) (width 0.6) (layer B.Cu) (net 2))
 (segment (start 114.5606 47.2203) (end 114.3 47.2203) (width 0.6) (layer B.Cu) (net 2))
 (segment (start 137.795 99.06) (end 136.0947 99.06) (width 0.6) (layer B.Cu) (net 11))
 (segment (start 121.285 62.865) (end 127.9663 69.5463) (width 0.6) (layer B.Cu) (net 11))
 (segment (start 127.9663 69.5463) (end 127.9663 90.9316) (width 0.6) (layer B.Cu) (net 11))
 (segment (start 127.9663 90.9316) (end 136.0947 99.06) (width 0.6) (layer B.Cu) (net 11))
 (segment (start 121.285 66.8053) (end 118.2367 69.8536) (width 0.6) (layer B.Cu) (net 27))
 (segment (start 118.2367 69.8536) (end 118.2367 77.9783) (width 0.6) (layer B.Cu) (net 27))
 (segment (start 118.2367 77.9783) (end 113.03 83.185) (width 0.6) (layer B.Cu) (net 27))
 (segment (start 121.285 65.405) (end 121.285 66.8053) (width 0.6) (layer B.Cu) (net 27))
 (segment (start 130.175 96.52) (end 128.4747 96.52) (width 0.6) (layer B.Cu) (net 19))
 (segment (start 121.285 69.85) (end 123.9543 72.5193) (width 0.6) (layer B.Cu) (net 19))
 (segment (start 123.9543 72.5193) (end 123.9543 91.9996) (width 0.6) (layer B.Cu) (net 19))
 (segment (start 123.9543 91.9996) (end 128.4747 96.52) (width 0.6) (layer B.Cu) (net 19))
 (segment (start 121.285 72.39) (end 121.285 73.7903) (width 0.6) (layer B.Cu) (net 26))
 (segment (start 121.285 73.7903) (end 119.8847 75.1906) (width 0.6) (layer B.Cu) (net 26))
 (segment (start 119.8847 75.1906) (end 119.8847 78.8703) (width 0.6) (layer B.Cu) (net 26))
 (segment (start 119.8847 78.8703) (end 113.03 85.725) (width 0.6) (layer B.Cu) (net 26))
 (segment (start 121.285 76.835) (end 125.7422 81.2922) (width 0.6) (layer F.Cu) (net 17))
 (segment (start 125.7422 81.2922) (end 125.7422 85.2343) (width 0.6) (layer F.Cu) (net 17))
 (segment (start 125.7422 85.2343) (end 128.4747 87.9668) (width 0.6) (layer F.Cu) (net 17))
 (segment (start 128.4747 87.9668) (end 128.4747 99.06) (width 0.6) (layer F.Cu) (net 17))
 (segment (start 130.175 99.06) (end 128.4747 99.06) (width 0.6) (layer F.Cu) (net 17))
 (segment (start 113.03 88.265) (end 114.3303 88.265) (width 0.6) (layer B.Cu) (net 25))
 (segment (start 121.285 79.375) (end 121.285 80.7753) (width 0.6) (layer B.Cu) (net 25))
 (segment (start 121.285 80.7753) (end 114.3303 87.73) (width 0.6) (layer B.Cu) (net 25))
 (segment (start 114.3303 87.73) (end 114.3303 88.265) (width 0.6) (layer B.Cu) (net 25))
 (segment (start 130.175 101.6) (end 128.4747 101.6) (width 0.6) (layer F.Cu) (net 16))
 (segment (start 121.285 83.82) (end 125.8436 88.3786) (width 0.6) (layer F.Cu) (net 16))
 (segment (start 125.8436 88.3786) (end 125.8436 98.9689) (width 0.6) (layer F.Cu) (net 16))
 (segment (start 125.8436 98.9689) (end 128.4747 101.6) (width 0.6) (layer F.Cu) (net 16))
 (segment (start 121.285 86.36) (end 119.8847 86.36) (width 0.6) (layer B.Cu) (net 24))
 (segment (start 119.8847 86.36) (end 115.4397 90.805) (width 0.6) (layer B.Cu) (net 24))
 (segment (start 115.4397 90.805) (end 113.03 90.805) (width 0.6) (layer B.Cu) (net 24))
 (segment (start 130.175 104.14) (end 128.4747 104.14) (width 0.6) (layer B.Cu) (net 15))
 (segment (start 121.285 90.805) (end 128.4747 97.9947) (width 0.6) (layer B.Cu) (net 15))
 (segment (start 128.4747 97.9947) (end 128.4747 104.14) (width 0.6) (layer B.Cu) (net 15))
 (segment (start 121.285 93.345) (end 113.03 93.345) (width 0.6) (layer B.Cu) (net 23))
 (segment (start 130.175 106.68) (end 128.4747 106.68) (width 0.6) (layer B.Cu) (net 14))
 (segment (start 121.285 97.79) (end 125.8436 102.3486) (width 0.6) (layer B.Cu) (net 14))
 (segment (start 125.8436 102.3486) (end 125.8436 104.0489) (width 0.6) (layer B.Cu) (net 14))
 (segment (start 125.8436 104.0489) (end 128.4747 106.68) (width 0.6) (layer B.Cu) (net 14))
 (segment (start 113.03 95.885) (end 114.3303 95.885) (width 0.6) (layer B.Cu) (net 22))
 (segment (start 121.285 100.33) (end 118.7753 100.33) (width 0.6) (layer B.Cu) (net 22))
 (segment (start 118.7753 100.33) (end 114.3303 95.885) (width 0.6) (layer B.Cu) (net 22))
 (segment (start 130.175 109.22) (end 128.4747 109.22) (width 0.6) (layer F.Cu) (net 13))
 (segment (start 121.285 104.775) (end 124.0297 104.775) (width 0.6) (layer F.Cu) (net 13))
 (segment (start 124.0297 104.775) (end 128.4747 109.22) (width 0.6) (layer F.Cu) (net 13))
 (segment (start 121.285 107.315) (end 113.03 99.06) (width 0.6) (layer B.Cu) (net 21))
 (segment (start 113.03 99.06) (end 113.03 98.425) (width 0.6) (layer B.Cu) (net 21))
 (segment (start 121.285 111.76) (end 130.175 111.76) (width 0.6) (layer B.Cu) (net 12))
 (segment (start 121.285 114.3) (end 113.03 106.045) (width 0.6) (layer B.Cu) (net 20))
 (segment (start 113.03 106.045) (end 113.03 100.965) (width 0.6) (layer B.Cu) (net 20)))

